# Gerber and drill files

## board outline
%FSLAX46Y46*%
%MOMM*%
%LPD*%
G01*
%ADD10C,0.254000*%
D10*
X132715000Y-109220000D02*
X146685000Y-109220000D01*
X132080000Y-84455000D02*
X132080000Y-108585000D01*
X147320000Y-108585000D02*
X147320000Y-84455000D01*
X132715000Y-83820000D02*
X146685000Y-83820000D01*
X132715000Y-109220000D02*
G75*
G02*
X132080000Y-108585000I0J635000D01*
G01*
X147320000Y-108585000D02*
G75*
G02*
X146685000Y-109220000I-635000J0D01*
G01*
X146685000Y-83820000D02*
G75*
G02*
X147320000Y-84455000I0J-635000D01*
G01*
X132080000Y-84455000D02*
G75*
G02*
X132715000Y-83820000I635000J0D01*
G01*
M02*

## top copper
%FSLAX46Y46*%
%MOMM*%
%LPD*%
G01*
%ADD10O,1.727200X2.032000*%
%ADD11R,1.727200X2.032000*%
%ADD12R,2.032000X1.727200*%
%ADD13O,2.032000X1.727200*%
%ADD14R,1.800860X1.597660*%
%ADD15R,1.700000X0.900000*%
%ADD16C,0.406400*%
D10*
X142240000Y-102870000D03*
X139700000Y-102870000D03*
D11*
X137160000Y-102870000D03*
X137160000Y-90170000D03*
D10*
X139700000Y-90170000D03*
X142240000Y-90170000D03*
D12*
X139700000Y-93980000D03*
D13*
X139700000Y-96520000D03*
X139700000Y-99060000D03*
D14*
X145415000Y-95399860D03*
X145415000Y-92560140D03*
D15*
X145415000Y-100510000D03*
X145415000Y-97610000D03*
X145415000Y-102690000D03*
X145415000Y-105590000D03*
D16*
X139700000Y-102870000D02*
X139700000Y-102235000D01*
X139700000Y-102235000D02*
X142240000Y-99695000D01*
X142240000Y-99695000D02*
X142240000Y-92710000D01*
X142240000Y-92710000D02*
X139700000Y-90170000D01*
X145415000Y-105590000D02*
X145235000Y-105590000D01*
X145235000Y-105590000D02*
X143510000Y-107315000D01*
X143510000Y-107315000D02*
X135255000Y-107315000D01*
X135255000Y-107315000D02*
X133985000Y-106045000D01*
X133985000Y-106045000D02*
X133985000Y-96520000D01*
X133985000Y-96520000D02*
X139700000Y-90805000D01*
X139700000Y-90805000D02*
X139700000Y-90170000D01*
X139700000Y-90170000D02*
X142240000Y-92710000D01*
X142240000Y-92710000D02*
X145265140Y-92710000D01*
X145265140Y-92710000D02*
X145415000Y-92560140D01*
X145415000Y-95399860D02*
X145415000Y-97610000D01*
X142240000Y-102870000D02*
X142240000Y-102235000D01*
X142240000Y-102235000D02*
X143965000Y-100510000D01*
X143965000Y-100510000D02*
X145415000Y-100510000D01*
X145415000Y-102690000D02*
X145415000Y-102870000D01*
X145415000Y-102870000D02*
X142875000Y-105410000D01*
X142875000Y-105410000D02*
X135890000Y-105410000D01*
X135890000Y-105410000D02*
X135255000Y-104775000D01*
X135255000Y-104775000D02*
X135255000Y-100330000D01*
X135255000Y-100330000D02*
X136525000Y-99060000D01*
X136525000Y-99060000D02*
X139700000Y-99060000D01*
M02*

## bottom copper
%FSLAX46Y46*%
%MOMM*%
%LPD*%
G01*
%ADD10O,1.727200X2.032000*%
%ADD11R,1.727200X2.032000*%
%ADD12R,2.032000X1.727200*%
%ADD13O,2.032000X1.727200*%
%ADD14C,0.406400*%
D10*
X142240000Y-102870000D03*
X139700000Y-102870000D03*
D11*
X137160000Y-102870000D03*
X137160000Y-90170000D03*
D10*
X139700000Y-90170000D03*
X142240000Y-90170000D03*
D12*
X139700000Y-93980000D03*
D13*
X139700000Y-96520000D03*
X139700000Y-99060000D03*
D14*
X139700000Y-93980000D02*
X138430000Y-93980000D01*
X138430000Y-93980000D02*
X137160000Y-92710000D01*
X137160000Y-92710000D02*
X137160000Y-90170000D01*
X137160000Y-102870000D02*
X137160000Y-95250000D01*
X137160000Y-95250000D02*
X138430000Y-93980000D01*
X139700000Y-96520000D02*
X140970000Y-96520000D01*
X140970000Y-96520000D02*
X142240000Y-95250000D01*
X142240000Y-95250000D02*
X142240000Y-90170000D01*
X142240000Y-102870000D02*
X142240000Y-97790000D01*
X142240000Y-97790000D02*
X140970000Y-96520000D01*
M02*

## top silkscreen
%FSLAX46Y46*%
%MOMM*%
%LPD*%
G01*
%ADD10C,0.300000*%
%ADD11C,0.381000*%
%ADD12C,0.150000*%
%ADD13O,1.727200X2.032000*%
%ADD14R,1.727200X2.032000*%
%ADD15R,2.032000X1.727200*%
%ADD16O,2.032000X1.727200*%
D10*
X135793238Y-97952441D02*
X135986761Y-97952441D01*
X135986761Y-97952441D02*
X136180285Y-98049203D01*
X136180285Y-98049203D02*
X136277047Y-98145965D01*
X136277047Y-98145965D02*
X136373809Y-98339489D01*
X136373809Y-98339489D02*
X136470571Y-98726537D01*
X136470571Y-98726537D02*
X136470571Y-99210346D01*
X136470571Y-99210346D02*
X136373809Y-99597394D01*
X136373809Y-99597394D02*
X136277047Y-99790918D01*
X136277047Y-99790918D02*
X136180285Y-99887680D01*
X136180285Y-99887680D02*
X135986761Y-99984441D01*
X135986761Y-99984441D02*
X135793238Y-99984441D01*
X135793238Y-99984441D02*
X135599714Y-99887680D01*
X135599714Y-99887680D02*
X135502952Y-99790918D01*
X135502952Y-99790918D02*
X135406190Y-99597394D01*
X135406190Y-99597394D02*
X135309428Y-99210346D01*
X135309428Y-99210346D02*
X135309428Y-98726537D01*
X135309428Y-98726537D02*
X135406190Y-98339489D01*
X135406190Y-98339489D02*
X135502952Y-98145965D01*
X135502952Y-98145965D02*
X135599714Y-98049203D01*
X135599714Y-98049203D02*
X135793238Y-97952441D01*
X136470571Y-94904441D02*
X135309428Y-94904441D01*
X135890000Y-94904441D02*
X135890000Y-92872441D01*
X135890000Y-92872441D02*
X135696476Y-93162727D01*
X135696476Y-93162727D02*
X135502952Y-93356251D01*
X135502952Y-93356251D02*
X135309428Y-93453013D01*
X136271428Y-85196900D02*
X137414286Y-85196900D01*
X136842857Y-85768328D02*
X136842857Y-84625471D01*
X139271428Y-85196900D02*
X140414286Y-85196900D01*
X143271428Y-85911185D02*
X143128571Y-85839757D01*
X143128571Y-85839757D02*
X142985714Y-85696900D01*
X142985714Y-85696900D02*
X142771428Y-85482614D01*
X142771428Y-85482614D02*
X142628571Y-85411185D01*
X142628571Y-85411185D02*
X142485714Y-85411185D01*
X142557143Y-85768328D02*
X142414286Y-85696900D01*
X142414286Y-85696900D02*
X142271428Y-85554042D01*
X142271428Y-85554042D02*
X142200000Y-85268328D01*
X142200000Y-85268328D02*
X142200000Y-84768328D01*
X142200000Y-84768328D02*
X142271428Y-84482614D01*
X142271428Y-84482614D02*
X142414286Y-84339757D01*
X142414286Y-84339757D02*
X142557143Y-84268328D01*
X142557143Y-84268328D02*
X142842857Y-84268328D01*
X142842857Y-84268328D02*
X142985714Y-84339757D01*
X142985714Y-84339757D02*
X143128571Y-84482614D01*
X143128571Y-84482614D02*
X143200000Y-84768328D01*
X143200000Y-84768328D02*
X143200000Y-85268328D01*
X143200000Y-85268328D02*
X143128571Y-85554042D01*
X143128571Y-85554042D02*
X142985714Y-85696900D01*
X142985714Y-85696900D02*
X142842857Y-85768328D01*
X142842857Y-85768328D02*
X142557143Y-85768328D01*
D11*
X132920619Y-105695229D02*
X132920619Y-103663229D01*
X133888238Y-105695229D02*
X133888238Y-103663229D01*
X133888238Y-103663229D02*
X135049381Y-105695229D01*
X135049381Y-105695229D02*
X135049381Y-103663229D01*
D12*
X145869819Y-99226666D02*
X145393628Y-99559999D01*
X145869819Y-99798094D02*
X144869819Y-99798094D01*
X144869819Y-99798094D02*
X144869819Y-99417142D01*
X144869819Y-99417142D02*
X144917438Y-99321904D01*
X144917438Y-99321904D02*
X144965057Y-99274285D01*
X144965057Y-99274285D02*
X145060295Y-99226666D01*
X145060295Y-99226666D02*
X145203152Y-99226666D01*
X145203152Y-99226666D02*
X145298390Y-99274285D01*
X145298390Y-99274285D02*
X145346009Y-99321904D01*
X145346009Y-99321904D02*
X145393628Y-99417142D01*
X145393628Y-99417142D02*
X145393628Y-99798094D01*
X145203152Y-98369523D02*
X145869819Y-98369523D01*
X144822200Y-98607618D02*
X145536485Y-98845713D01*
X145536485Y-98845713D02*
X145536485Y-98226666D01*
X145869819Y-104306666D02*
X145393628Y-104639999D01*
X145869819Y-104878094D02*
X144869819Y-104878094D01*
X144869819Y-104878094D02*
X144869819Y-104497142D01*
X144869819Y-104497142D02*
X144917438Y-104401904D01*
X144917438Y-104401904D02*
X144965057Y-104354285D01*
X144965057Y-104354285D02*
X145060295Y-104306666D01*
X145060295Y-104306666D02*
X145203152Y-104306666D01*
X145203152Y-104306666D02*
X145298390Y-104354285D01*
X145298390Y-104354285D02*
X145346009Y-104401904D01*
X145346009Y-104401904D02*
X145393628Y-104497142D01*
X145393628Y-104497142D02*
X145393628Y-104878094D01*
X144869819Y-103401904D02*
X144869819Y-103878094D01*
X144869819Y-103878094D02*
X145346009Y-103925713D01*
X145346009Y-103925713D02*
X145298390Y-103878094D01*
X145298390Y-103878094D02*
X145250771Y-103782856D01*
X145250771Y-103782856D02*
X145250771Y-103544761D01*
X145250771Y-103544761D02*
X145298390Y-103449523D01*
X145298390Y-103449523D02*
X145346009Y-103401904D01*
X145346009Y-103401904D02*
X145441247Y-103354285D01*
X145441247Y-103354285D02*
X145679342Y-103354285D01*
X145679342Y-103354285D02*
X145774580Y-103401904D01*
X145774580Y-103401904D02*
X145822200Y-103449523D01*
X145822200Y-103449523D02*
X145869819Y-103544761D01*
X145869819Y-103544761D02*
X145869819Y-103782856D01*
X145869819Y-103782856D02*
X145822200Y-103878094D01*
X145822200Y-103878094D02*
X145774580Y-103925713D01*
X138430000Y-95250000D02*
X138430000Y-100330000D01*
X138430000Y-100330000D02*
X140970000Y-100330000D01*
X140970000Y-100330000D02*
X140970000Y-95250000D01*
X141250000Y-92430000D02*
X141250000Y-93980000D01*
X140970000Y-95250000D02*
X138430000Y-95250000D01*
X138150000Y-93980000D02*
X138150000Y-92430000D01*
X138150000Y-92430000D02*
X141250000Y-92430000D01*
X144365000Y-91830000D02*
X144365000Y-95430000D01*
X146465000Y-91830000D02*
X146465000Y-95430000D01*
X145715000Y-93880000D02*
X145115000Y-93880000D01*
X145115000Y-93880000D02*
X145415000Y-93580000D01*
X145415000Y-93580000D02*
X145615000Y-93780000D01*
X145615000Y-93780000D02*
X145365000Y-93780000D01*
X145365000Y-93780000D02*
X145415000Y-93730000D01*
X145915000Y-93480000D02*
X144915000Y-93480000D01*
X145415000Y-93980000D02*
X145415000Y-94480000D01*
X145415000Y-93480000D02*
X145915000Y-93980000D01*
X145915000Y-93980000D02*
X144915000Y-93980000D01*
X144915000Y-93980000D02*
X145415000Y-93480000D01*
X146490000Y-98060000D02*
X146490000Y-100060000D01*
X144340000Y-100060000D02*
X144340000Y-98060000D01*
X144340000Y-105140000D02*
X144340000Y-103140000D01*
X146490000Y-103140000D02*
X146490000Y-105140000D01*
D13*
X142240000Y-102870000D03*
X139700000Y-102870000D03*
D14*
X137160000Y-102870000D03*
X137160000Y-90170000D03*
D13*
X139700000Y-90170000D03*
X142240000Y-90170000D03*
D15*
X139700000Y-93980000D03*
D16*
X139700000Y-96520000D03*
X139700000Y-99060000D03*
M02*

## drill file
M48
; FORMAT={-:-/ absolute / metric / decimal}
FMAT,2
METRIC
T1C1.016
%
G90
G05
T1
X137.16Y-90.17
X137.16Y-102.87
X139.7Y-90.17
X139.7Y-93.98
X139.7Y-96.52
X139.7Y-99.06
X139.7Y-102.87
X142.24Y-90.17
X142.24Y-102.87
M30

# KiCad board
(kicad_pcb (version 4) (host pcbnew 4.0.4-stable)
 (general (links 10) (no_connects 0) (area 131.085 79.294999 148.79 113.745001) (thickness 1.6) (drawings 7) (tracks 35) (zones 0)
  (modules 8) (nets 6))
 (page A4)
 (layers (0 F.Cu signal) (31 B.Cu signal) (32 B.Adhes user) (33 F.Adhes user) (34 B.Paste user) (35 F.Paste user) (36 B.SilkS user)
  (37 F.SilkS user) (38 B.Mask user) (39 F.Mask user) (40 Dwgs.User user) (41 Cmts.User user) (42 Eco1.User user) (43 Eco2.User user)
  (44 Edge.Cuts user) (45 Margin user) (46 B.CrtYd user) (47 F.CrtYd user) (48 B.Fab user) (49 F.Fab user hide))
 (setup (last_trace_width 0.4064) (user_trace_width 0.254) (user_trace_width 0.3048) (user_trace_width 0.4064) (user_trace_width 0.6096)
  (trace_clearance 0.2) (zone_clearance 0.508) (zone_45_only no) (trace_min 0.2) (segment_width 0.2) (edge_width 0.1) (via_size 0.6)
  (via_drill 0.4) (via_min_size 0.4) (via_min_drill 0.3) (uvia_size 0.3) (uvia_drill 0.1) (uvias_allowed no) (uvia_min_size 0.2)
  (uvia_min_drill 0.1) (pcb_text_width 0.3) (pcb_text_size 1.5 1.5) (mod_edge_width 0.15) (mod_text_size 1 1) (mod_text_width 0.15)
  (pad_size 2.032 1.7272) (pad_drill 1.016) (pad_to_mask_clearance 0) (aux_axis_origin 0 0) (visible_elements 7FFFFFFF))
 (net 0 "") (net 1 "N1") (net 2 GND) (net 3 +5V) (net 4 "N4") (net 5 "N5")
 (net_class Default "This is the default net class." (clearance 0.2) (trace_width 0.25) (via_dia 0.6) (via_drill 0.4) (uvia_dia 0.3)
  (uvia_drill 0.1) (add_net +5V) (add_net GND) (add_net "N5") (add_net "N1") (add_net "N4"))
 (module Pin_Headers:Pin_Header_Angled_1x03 (layer F.Cu) (at 142.24 102.87 270)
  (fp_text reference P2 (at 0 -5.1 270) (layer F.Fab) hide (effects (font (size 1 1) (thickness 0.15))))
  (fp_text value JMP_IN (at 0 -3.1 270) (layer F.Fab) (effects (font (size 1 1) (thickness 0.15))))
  (pad 1 thru_hole oval (at 0 0 270) (size 2.032 1.7272) (drill 1.016) (layers *.Cu *.Mask F.SilkS) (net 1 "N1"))
  (pad 2 thru_hole oval (at 0 2.54 270) (size 2.032 1.7272) (drill 1.016) (layers *.Cu *.Mask F.SilkS) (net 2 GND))
  (pad 3 thru_hole rect (at 0 5.08 270) (size 2.032 1.7272) (drill 1.016) (layers *.Cu *.Mask F.SilkS) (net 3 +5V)))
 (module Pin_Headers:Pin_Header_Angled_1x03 (layer F.Cu) (at 137.16 90.17 90)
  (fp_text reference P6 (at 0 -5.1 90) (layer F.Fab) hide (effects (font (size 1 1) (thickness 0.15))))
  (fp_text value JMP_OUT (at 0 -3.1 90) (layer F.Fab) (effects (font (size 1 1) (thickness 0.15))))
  (pad 1 thru_hole rect (at 0 0 90) (size 2.032 1.7272) (drill 1.016) (layers *.Cu *.Mask F.SilkS) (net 3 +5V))
  (pad 2 thru_hole oval (at 0 2.54 90) (size 2.032 1.7272) (drill 1.016) (layers *.Cu *.Mask F.SilkS) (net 2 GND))
  (pad 3 thru_hole oval (at 0 5.08 90) (size 2.032 1.7272) (drill 1.016) (layers *.Cu *.Mask F.SilkS) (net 1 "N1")))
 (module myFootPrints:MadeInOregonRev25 (layer F.Cu) (at 144.145 96.52 90)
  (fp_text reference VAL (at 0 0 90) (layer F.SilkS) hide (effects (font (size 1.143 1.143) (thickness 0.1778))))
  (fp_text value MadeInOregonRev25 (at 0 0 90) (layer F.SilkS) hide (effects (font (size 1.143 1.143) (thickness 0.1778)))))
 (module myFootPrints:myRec (layer F.Cu) (at 139.7 96.52)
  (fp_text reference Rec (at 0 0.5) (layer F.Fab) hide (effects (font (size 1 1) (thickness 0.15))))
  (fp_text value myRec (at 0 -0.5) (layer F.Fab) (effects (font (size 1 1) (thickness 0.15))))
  (fp_line (start -6.985 12.7) (end 6.985 12.7) (layer Edge.Cuts) (width 0.254))
  (fp_line (start -7.62 -12.065) (end -7.62 12.065) (layer Edge.Cuts) (width 0.254))
  (fp_line (start 7.62 12.065) (end 7.62 -12.065) (layer Edge.Cuts) (width 0.254))
  (fp_line (start -6.985 -12.7) (end 6.985 -12.7) (layer Edge.Cuts) (width 0.254))
  (fp_arc (start -6.985 12.065) (end -6.985 12.7) (angle 90) (layer Edge.Cuts) (width 0.254))
  (fp_arc (start 6.985 12.065) (end 7.62 12.065) (angle 90) (layer Edge.Cuts) (width 0.254))
  (fp_arc (start 6.985 -12.065) (end 6.985 -12.7) (angle 90) (layer Edge.Cuts) (width 0.254))
  (fp_arc (start -6.985 -12.065) (end -7.62 -12.065) (angle 90) (layer Edge.Cuts) (width 0.254)))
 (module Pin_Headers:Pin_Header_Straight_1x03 (layer F.Cu) (at 139.7 93.98)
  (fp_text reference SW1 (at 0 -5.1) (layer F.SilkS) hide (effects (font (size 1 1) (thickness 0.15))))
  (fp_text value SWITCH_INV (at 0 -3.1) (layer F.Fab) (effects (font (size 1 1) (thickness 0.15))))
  (fp_line (start -1.27 1.27) (end -1.27 6.35) (layer F.SilkS) (width 0.15))
  (fp_line (start -1.27 6.35) (end 1.27 6.35) (layer F.SilkS) (width 0.15))
  (fp_line (start 1.27 6.35) (end 1.27 1.27) (layer F.SilkS) (width 0.15))
  (fp_line (start 1.55 -1.55) (end 1.55 0) (layer F.SilkS) (width 0.15))
  (fp_line (start 1.27 1.27) (end -1.27 1.27) (layer F.SilkS) (width 0.15))
  (fp_line (start -1.55 0) (end -1.55 -1.55) (layer F.SilkS) (width 0.15))
  (fp_line (start -1.55 -1.55) (end 1.55 -1.55) (layer F.SilkS) (width 0.15))
  (pad 1 thru_hole rect (at 0 0) (size 2.032 1.7272) (drill 1.016) (layers *.Cu *.Mask F.SilkS) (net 3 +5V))
  (pad 2 thru_hole oval (at 0 2.54) (size 2.032 1.7272) (drill 1.016) (layers *.Cu *.Mask F.SilkS) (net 1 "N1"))
  (pad 3 thru_hole oval (at 0 5.08) (size 2.032 1.7272) (drill 1.016) (layers *.Cu *.Mask F.SilkS) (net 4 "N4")))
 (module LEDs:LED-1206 (layer F.Cu) (at 145.415 93.98 270)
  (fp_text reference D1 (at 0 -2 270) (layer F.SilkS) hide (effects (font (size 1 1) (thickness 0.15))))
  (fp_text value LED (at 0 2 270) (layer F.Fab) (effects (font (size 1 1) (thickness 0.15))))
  (fp_line (start -2.15 1.05) (end 1.45 1.05) (layer F.SilkS) (width 0.15))
  (fp_line (start -2.15 -1.05) (end 1.45 -1.05) (layer F.SilkS) (width 0.15))
  (fp_line (start -0.1 -0.3) (end -0.1 0.3) (layer F.SilkS) (width 0.15))
  (fp_line (start -0.1 0.3) (end -0.4 0) (layer F.SilkS) (width 0.15))
  (fp_line (start -0.4 0) (end -0.2 -0.2) (layer F.SilkS) (width 0.15))
  (fp_line (start -0.2 -0.2) (end -0.2 0.05) (layer F.SilkS) (width 0.15))
  (fp_line (start -0.2 0.05) (end -0.25 0) (layer F.SilkS) (width 0.15))
  (fp_line (start -0.5 -0.5) (end -0.5 0.5) (layer F.SilkS) (width 0.15))
  (fp_line (start 0 0) (end 0.5 0) (layer F.SilkS) (width 0.15))
  (fp_line (start -0.5 0) (end 0 -0.5) (layer F.SilkS) (width 0.15))
  (fp_line (start 0 -0.5) (end 0 0.5) (layer F.SilkS) (width 0.15))
  (fp_line (start 0 0.5) (end -0.5 0) (layer F.SilkS) (width 0.15))
  (pad 2 smd rect (at 1.41986 0 90) (size 1.59766 1.80086) (layers F.Cu F.Paste F.Mask) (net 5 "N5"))
  (pad 1 smd rect (at -1.41986 0 90) (size 1.59766 1.80086) (layers F.Cu F.Paste F.Mask) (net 2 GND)))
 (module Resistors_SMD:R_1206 (layer F.Cu) (at 145.415 99.06 90)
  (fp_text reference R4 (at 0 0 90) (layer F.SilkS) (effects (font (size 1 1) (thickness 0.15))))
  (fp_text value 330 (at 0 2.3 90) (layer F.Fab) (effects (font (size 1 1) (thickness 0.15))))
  (fp_line (start 1 1.075) (end -1 1.075) (layer F.SilkS) (width 0.15))
  (fp_line (start -1 -1.075) (end 1 -1.075) (layer F.SilkS) (width 0.15))
  (pad 1 smd rect (at -1.45 0 90) (size 0.9 1.7) (layers F.Cu F.Paste F.Mask) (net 1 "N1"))
  (pad 2 smd rect (at 1.45 0 90) (size 0.9 1.7) (layers F.Cu F.Paste F.Mask) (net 5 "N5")))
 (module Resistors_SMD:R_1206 (layer F.Cu) (at 145.415 104.14 270)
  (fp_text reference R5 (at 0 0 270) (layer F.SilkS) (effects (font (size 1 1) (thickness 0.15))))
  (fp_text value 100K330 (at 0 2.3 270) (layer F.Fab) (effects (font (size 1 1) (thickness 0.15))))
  (fp_line (start 1 1.075) (end -1 1.075) (layer F.SilkS) (width 0.15))
  (fp_line (start -1 -1.075) (end 1 -1.075) (layer F.SilkS) (width 0.15))
  (pad 1 smd rect (at -1.45 0 270) (size 0.9 1.7) (layers F.Cu F.Paste F.Mask) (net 4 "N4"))
  (pad 2 smd rect (at 1.45 0 270) (size 0.9 1.7) (layers F.Cu F.Paste F.Mask) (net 2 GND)))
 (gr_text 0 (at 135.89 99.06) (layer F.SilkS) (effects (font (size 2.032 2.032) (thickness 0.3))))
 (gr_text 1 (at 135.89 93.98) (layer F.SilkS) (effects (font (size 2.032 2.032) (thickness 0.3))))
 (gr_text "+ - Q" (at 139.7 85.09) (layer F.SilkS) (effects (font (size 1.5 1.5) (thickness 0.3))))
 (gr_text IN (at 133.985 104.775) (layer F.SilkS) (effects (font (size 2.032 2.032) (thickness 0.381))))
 (segment (start 139.7 102.87) (end 139.7 102.235) (width 0.4064) (layer F.Cu) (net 2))
 (segment (start 139.7 102.235) (end 142.24 99.695) (width 0.4064) (layer F.Cu) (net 2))
 (segment (start 142.24 99.695) (end 142.24 92.71) (width 0.4064) (layer F.Cu) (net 2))
 (segment (start 142.24 92.71) (end 139.7 90.17) (width 0.4064) (layer F.Cu) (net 2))
 (segment (start 145.415 105.59) (end 145.235 105.59) (width 0.4064) (layer F.Cu) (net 2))
 (segment (start 145.235 105.59) (end 143.51 107.315) (width 0.4064) (layer F.Cu) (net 2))
 (segment (start 143.51 107.315) (end 135.255 107.315) (width 0.4064) (layer F.Cu) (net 2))
 (segment (start 135.255 107.315) (end 133.985 106.045) (width 0.4064) (layer F.Cu) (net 2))
 (segment (start 133.985 106.045) (end 133.985 96.52) (width 0.4064) (layer F.Cu) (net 2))
 (segment (start 133.985 96.52) (end 139.7 90.805) (width 0.4064) (layer F.Cu) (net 2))
 (segment (start 139.7 90.805) (end 139.7 90.17) (width 0.4064) (layer F.Cu) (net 2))
 (segment (start 139.7 90.17) (end 142.24 92.71) (width 0.4064) (layer F.Cu) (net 2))
 (segment (start 142.24 92.71) (end 145.26514 92.71) (width 0.4064) (layer F.Cu) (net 2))
 (segment (start 145.26514 92.71) (end 145.415 92.56014) (width 0.4064) (layer F.Cu) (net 2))
 (segment (start 145.415 95.39986) (end 145.415 97.61) (width 0.4064) (layer F.Cu) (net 5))
 (segment (start 139.7 93.98) (end 138.43 93.98) (width 0.4064) (layer B.Cu) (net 3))
 (segment (start 138.43 93.98) (end 137.16 92.71) (width 0.4064) (layer B.Cu) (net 3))
 (segment (start 137.16 92.71) (end 137.16 90.17) (width 0.4064) (layer B.Cu) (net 3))
 (segment (start 137.16 102.87) (end 137.16 95.25) (width 0.4064) (layer B.Cu) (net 3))
 (segment (start 137.16 95.25) (end 138.43 93.98) (width 0.4064) (layer B.Cu) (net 3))
 (segment (start 142.24 102.87) (end 142.24 102.235) (width 0.4064) (layer F.Cu) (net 1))
 (segment (start 142.24 102.235) (end 143.965 100.51) (width 0.4064) (layer F.Cu) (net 1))
 (segment (start 143.965 100.51) (end 145.415 100.51) (width 0.4064) (layer F.Cu) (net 1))
 (segment (start 139.7 96.52) (end 140.97 96.52) (width 0.4064) (layer B.Cu) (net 1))
 (segment (start 140.97 96.52) (end 142.24 95.25) (width 0.4064) (layer B.Cu) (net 1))
 (segment (start 142.24 95.25) (end 142.24 90.17) (width 0.4064) (layer B.Cu) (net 1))
 (segment (start 142.24 102.87) (end 142.24 97.79) (width 0.4064) (layer B.Cu) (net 1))
 (segment (start 142.24 97.79) (end 140.97 96.52) (width 0.4064) (layer B.Cu) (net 1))
 (segment (start 145.415 102.69) (end 145.415 102.87) (width 0.4064) (layer F.Cu) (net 4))
 (segment (start 145.415 102.87) (end 142.875 105.41) (width 0.4064) (layer F.Cu) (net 4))
 (segment (start 142.875 105.41) (end 135.89 105.41) (width 0.4064) (layer F.Cu) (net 4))
 (segment (start 135.89 105.41) (end 135.255 104.775) (width 0.4064) (layer F.Cu) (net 4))
 (segment (start 135.255 104.775) (end 135.255 100.33) (width 0.4064) (layer F.Cu) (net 4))
 (segment (start 135.255 100.33) (end 136.525 99.06) (width 0.4064) (layer F.Cu) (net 4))
 (segment (start 136.525 99.06) (end 139.7 99.06) (width 0.4064) (layer F.Cu) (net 4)))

